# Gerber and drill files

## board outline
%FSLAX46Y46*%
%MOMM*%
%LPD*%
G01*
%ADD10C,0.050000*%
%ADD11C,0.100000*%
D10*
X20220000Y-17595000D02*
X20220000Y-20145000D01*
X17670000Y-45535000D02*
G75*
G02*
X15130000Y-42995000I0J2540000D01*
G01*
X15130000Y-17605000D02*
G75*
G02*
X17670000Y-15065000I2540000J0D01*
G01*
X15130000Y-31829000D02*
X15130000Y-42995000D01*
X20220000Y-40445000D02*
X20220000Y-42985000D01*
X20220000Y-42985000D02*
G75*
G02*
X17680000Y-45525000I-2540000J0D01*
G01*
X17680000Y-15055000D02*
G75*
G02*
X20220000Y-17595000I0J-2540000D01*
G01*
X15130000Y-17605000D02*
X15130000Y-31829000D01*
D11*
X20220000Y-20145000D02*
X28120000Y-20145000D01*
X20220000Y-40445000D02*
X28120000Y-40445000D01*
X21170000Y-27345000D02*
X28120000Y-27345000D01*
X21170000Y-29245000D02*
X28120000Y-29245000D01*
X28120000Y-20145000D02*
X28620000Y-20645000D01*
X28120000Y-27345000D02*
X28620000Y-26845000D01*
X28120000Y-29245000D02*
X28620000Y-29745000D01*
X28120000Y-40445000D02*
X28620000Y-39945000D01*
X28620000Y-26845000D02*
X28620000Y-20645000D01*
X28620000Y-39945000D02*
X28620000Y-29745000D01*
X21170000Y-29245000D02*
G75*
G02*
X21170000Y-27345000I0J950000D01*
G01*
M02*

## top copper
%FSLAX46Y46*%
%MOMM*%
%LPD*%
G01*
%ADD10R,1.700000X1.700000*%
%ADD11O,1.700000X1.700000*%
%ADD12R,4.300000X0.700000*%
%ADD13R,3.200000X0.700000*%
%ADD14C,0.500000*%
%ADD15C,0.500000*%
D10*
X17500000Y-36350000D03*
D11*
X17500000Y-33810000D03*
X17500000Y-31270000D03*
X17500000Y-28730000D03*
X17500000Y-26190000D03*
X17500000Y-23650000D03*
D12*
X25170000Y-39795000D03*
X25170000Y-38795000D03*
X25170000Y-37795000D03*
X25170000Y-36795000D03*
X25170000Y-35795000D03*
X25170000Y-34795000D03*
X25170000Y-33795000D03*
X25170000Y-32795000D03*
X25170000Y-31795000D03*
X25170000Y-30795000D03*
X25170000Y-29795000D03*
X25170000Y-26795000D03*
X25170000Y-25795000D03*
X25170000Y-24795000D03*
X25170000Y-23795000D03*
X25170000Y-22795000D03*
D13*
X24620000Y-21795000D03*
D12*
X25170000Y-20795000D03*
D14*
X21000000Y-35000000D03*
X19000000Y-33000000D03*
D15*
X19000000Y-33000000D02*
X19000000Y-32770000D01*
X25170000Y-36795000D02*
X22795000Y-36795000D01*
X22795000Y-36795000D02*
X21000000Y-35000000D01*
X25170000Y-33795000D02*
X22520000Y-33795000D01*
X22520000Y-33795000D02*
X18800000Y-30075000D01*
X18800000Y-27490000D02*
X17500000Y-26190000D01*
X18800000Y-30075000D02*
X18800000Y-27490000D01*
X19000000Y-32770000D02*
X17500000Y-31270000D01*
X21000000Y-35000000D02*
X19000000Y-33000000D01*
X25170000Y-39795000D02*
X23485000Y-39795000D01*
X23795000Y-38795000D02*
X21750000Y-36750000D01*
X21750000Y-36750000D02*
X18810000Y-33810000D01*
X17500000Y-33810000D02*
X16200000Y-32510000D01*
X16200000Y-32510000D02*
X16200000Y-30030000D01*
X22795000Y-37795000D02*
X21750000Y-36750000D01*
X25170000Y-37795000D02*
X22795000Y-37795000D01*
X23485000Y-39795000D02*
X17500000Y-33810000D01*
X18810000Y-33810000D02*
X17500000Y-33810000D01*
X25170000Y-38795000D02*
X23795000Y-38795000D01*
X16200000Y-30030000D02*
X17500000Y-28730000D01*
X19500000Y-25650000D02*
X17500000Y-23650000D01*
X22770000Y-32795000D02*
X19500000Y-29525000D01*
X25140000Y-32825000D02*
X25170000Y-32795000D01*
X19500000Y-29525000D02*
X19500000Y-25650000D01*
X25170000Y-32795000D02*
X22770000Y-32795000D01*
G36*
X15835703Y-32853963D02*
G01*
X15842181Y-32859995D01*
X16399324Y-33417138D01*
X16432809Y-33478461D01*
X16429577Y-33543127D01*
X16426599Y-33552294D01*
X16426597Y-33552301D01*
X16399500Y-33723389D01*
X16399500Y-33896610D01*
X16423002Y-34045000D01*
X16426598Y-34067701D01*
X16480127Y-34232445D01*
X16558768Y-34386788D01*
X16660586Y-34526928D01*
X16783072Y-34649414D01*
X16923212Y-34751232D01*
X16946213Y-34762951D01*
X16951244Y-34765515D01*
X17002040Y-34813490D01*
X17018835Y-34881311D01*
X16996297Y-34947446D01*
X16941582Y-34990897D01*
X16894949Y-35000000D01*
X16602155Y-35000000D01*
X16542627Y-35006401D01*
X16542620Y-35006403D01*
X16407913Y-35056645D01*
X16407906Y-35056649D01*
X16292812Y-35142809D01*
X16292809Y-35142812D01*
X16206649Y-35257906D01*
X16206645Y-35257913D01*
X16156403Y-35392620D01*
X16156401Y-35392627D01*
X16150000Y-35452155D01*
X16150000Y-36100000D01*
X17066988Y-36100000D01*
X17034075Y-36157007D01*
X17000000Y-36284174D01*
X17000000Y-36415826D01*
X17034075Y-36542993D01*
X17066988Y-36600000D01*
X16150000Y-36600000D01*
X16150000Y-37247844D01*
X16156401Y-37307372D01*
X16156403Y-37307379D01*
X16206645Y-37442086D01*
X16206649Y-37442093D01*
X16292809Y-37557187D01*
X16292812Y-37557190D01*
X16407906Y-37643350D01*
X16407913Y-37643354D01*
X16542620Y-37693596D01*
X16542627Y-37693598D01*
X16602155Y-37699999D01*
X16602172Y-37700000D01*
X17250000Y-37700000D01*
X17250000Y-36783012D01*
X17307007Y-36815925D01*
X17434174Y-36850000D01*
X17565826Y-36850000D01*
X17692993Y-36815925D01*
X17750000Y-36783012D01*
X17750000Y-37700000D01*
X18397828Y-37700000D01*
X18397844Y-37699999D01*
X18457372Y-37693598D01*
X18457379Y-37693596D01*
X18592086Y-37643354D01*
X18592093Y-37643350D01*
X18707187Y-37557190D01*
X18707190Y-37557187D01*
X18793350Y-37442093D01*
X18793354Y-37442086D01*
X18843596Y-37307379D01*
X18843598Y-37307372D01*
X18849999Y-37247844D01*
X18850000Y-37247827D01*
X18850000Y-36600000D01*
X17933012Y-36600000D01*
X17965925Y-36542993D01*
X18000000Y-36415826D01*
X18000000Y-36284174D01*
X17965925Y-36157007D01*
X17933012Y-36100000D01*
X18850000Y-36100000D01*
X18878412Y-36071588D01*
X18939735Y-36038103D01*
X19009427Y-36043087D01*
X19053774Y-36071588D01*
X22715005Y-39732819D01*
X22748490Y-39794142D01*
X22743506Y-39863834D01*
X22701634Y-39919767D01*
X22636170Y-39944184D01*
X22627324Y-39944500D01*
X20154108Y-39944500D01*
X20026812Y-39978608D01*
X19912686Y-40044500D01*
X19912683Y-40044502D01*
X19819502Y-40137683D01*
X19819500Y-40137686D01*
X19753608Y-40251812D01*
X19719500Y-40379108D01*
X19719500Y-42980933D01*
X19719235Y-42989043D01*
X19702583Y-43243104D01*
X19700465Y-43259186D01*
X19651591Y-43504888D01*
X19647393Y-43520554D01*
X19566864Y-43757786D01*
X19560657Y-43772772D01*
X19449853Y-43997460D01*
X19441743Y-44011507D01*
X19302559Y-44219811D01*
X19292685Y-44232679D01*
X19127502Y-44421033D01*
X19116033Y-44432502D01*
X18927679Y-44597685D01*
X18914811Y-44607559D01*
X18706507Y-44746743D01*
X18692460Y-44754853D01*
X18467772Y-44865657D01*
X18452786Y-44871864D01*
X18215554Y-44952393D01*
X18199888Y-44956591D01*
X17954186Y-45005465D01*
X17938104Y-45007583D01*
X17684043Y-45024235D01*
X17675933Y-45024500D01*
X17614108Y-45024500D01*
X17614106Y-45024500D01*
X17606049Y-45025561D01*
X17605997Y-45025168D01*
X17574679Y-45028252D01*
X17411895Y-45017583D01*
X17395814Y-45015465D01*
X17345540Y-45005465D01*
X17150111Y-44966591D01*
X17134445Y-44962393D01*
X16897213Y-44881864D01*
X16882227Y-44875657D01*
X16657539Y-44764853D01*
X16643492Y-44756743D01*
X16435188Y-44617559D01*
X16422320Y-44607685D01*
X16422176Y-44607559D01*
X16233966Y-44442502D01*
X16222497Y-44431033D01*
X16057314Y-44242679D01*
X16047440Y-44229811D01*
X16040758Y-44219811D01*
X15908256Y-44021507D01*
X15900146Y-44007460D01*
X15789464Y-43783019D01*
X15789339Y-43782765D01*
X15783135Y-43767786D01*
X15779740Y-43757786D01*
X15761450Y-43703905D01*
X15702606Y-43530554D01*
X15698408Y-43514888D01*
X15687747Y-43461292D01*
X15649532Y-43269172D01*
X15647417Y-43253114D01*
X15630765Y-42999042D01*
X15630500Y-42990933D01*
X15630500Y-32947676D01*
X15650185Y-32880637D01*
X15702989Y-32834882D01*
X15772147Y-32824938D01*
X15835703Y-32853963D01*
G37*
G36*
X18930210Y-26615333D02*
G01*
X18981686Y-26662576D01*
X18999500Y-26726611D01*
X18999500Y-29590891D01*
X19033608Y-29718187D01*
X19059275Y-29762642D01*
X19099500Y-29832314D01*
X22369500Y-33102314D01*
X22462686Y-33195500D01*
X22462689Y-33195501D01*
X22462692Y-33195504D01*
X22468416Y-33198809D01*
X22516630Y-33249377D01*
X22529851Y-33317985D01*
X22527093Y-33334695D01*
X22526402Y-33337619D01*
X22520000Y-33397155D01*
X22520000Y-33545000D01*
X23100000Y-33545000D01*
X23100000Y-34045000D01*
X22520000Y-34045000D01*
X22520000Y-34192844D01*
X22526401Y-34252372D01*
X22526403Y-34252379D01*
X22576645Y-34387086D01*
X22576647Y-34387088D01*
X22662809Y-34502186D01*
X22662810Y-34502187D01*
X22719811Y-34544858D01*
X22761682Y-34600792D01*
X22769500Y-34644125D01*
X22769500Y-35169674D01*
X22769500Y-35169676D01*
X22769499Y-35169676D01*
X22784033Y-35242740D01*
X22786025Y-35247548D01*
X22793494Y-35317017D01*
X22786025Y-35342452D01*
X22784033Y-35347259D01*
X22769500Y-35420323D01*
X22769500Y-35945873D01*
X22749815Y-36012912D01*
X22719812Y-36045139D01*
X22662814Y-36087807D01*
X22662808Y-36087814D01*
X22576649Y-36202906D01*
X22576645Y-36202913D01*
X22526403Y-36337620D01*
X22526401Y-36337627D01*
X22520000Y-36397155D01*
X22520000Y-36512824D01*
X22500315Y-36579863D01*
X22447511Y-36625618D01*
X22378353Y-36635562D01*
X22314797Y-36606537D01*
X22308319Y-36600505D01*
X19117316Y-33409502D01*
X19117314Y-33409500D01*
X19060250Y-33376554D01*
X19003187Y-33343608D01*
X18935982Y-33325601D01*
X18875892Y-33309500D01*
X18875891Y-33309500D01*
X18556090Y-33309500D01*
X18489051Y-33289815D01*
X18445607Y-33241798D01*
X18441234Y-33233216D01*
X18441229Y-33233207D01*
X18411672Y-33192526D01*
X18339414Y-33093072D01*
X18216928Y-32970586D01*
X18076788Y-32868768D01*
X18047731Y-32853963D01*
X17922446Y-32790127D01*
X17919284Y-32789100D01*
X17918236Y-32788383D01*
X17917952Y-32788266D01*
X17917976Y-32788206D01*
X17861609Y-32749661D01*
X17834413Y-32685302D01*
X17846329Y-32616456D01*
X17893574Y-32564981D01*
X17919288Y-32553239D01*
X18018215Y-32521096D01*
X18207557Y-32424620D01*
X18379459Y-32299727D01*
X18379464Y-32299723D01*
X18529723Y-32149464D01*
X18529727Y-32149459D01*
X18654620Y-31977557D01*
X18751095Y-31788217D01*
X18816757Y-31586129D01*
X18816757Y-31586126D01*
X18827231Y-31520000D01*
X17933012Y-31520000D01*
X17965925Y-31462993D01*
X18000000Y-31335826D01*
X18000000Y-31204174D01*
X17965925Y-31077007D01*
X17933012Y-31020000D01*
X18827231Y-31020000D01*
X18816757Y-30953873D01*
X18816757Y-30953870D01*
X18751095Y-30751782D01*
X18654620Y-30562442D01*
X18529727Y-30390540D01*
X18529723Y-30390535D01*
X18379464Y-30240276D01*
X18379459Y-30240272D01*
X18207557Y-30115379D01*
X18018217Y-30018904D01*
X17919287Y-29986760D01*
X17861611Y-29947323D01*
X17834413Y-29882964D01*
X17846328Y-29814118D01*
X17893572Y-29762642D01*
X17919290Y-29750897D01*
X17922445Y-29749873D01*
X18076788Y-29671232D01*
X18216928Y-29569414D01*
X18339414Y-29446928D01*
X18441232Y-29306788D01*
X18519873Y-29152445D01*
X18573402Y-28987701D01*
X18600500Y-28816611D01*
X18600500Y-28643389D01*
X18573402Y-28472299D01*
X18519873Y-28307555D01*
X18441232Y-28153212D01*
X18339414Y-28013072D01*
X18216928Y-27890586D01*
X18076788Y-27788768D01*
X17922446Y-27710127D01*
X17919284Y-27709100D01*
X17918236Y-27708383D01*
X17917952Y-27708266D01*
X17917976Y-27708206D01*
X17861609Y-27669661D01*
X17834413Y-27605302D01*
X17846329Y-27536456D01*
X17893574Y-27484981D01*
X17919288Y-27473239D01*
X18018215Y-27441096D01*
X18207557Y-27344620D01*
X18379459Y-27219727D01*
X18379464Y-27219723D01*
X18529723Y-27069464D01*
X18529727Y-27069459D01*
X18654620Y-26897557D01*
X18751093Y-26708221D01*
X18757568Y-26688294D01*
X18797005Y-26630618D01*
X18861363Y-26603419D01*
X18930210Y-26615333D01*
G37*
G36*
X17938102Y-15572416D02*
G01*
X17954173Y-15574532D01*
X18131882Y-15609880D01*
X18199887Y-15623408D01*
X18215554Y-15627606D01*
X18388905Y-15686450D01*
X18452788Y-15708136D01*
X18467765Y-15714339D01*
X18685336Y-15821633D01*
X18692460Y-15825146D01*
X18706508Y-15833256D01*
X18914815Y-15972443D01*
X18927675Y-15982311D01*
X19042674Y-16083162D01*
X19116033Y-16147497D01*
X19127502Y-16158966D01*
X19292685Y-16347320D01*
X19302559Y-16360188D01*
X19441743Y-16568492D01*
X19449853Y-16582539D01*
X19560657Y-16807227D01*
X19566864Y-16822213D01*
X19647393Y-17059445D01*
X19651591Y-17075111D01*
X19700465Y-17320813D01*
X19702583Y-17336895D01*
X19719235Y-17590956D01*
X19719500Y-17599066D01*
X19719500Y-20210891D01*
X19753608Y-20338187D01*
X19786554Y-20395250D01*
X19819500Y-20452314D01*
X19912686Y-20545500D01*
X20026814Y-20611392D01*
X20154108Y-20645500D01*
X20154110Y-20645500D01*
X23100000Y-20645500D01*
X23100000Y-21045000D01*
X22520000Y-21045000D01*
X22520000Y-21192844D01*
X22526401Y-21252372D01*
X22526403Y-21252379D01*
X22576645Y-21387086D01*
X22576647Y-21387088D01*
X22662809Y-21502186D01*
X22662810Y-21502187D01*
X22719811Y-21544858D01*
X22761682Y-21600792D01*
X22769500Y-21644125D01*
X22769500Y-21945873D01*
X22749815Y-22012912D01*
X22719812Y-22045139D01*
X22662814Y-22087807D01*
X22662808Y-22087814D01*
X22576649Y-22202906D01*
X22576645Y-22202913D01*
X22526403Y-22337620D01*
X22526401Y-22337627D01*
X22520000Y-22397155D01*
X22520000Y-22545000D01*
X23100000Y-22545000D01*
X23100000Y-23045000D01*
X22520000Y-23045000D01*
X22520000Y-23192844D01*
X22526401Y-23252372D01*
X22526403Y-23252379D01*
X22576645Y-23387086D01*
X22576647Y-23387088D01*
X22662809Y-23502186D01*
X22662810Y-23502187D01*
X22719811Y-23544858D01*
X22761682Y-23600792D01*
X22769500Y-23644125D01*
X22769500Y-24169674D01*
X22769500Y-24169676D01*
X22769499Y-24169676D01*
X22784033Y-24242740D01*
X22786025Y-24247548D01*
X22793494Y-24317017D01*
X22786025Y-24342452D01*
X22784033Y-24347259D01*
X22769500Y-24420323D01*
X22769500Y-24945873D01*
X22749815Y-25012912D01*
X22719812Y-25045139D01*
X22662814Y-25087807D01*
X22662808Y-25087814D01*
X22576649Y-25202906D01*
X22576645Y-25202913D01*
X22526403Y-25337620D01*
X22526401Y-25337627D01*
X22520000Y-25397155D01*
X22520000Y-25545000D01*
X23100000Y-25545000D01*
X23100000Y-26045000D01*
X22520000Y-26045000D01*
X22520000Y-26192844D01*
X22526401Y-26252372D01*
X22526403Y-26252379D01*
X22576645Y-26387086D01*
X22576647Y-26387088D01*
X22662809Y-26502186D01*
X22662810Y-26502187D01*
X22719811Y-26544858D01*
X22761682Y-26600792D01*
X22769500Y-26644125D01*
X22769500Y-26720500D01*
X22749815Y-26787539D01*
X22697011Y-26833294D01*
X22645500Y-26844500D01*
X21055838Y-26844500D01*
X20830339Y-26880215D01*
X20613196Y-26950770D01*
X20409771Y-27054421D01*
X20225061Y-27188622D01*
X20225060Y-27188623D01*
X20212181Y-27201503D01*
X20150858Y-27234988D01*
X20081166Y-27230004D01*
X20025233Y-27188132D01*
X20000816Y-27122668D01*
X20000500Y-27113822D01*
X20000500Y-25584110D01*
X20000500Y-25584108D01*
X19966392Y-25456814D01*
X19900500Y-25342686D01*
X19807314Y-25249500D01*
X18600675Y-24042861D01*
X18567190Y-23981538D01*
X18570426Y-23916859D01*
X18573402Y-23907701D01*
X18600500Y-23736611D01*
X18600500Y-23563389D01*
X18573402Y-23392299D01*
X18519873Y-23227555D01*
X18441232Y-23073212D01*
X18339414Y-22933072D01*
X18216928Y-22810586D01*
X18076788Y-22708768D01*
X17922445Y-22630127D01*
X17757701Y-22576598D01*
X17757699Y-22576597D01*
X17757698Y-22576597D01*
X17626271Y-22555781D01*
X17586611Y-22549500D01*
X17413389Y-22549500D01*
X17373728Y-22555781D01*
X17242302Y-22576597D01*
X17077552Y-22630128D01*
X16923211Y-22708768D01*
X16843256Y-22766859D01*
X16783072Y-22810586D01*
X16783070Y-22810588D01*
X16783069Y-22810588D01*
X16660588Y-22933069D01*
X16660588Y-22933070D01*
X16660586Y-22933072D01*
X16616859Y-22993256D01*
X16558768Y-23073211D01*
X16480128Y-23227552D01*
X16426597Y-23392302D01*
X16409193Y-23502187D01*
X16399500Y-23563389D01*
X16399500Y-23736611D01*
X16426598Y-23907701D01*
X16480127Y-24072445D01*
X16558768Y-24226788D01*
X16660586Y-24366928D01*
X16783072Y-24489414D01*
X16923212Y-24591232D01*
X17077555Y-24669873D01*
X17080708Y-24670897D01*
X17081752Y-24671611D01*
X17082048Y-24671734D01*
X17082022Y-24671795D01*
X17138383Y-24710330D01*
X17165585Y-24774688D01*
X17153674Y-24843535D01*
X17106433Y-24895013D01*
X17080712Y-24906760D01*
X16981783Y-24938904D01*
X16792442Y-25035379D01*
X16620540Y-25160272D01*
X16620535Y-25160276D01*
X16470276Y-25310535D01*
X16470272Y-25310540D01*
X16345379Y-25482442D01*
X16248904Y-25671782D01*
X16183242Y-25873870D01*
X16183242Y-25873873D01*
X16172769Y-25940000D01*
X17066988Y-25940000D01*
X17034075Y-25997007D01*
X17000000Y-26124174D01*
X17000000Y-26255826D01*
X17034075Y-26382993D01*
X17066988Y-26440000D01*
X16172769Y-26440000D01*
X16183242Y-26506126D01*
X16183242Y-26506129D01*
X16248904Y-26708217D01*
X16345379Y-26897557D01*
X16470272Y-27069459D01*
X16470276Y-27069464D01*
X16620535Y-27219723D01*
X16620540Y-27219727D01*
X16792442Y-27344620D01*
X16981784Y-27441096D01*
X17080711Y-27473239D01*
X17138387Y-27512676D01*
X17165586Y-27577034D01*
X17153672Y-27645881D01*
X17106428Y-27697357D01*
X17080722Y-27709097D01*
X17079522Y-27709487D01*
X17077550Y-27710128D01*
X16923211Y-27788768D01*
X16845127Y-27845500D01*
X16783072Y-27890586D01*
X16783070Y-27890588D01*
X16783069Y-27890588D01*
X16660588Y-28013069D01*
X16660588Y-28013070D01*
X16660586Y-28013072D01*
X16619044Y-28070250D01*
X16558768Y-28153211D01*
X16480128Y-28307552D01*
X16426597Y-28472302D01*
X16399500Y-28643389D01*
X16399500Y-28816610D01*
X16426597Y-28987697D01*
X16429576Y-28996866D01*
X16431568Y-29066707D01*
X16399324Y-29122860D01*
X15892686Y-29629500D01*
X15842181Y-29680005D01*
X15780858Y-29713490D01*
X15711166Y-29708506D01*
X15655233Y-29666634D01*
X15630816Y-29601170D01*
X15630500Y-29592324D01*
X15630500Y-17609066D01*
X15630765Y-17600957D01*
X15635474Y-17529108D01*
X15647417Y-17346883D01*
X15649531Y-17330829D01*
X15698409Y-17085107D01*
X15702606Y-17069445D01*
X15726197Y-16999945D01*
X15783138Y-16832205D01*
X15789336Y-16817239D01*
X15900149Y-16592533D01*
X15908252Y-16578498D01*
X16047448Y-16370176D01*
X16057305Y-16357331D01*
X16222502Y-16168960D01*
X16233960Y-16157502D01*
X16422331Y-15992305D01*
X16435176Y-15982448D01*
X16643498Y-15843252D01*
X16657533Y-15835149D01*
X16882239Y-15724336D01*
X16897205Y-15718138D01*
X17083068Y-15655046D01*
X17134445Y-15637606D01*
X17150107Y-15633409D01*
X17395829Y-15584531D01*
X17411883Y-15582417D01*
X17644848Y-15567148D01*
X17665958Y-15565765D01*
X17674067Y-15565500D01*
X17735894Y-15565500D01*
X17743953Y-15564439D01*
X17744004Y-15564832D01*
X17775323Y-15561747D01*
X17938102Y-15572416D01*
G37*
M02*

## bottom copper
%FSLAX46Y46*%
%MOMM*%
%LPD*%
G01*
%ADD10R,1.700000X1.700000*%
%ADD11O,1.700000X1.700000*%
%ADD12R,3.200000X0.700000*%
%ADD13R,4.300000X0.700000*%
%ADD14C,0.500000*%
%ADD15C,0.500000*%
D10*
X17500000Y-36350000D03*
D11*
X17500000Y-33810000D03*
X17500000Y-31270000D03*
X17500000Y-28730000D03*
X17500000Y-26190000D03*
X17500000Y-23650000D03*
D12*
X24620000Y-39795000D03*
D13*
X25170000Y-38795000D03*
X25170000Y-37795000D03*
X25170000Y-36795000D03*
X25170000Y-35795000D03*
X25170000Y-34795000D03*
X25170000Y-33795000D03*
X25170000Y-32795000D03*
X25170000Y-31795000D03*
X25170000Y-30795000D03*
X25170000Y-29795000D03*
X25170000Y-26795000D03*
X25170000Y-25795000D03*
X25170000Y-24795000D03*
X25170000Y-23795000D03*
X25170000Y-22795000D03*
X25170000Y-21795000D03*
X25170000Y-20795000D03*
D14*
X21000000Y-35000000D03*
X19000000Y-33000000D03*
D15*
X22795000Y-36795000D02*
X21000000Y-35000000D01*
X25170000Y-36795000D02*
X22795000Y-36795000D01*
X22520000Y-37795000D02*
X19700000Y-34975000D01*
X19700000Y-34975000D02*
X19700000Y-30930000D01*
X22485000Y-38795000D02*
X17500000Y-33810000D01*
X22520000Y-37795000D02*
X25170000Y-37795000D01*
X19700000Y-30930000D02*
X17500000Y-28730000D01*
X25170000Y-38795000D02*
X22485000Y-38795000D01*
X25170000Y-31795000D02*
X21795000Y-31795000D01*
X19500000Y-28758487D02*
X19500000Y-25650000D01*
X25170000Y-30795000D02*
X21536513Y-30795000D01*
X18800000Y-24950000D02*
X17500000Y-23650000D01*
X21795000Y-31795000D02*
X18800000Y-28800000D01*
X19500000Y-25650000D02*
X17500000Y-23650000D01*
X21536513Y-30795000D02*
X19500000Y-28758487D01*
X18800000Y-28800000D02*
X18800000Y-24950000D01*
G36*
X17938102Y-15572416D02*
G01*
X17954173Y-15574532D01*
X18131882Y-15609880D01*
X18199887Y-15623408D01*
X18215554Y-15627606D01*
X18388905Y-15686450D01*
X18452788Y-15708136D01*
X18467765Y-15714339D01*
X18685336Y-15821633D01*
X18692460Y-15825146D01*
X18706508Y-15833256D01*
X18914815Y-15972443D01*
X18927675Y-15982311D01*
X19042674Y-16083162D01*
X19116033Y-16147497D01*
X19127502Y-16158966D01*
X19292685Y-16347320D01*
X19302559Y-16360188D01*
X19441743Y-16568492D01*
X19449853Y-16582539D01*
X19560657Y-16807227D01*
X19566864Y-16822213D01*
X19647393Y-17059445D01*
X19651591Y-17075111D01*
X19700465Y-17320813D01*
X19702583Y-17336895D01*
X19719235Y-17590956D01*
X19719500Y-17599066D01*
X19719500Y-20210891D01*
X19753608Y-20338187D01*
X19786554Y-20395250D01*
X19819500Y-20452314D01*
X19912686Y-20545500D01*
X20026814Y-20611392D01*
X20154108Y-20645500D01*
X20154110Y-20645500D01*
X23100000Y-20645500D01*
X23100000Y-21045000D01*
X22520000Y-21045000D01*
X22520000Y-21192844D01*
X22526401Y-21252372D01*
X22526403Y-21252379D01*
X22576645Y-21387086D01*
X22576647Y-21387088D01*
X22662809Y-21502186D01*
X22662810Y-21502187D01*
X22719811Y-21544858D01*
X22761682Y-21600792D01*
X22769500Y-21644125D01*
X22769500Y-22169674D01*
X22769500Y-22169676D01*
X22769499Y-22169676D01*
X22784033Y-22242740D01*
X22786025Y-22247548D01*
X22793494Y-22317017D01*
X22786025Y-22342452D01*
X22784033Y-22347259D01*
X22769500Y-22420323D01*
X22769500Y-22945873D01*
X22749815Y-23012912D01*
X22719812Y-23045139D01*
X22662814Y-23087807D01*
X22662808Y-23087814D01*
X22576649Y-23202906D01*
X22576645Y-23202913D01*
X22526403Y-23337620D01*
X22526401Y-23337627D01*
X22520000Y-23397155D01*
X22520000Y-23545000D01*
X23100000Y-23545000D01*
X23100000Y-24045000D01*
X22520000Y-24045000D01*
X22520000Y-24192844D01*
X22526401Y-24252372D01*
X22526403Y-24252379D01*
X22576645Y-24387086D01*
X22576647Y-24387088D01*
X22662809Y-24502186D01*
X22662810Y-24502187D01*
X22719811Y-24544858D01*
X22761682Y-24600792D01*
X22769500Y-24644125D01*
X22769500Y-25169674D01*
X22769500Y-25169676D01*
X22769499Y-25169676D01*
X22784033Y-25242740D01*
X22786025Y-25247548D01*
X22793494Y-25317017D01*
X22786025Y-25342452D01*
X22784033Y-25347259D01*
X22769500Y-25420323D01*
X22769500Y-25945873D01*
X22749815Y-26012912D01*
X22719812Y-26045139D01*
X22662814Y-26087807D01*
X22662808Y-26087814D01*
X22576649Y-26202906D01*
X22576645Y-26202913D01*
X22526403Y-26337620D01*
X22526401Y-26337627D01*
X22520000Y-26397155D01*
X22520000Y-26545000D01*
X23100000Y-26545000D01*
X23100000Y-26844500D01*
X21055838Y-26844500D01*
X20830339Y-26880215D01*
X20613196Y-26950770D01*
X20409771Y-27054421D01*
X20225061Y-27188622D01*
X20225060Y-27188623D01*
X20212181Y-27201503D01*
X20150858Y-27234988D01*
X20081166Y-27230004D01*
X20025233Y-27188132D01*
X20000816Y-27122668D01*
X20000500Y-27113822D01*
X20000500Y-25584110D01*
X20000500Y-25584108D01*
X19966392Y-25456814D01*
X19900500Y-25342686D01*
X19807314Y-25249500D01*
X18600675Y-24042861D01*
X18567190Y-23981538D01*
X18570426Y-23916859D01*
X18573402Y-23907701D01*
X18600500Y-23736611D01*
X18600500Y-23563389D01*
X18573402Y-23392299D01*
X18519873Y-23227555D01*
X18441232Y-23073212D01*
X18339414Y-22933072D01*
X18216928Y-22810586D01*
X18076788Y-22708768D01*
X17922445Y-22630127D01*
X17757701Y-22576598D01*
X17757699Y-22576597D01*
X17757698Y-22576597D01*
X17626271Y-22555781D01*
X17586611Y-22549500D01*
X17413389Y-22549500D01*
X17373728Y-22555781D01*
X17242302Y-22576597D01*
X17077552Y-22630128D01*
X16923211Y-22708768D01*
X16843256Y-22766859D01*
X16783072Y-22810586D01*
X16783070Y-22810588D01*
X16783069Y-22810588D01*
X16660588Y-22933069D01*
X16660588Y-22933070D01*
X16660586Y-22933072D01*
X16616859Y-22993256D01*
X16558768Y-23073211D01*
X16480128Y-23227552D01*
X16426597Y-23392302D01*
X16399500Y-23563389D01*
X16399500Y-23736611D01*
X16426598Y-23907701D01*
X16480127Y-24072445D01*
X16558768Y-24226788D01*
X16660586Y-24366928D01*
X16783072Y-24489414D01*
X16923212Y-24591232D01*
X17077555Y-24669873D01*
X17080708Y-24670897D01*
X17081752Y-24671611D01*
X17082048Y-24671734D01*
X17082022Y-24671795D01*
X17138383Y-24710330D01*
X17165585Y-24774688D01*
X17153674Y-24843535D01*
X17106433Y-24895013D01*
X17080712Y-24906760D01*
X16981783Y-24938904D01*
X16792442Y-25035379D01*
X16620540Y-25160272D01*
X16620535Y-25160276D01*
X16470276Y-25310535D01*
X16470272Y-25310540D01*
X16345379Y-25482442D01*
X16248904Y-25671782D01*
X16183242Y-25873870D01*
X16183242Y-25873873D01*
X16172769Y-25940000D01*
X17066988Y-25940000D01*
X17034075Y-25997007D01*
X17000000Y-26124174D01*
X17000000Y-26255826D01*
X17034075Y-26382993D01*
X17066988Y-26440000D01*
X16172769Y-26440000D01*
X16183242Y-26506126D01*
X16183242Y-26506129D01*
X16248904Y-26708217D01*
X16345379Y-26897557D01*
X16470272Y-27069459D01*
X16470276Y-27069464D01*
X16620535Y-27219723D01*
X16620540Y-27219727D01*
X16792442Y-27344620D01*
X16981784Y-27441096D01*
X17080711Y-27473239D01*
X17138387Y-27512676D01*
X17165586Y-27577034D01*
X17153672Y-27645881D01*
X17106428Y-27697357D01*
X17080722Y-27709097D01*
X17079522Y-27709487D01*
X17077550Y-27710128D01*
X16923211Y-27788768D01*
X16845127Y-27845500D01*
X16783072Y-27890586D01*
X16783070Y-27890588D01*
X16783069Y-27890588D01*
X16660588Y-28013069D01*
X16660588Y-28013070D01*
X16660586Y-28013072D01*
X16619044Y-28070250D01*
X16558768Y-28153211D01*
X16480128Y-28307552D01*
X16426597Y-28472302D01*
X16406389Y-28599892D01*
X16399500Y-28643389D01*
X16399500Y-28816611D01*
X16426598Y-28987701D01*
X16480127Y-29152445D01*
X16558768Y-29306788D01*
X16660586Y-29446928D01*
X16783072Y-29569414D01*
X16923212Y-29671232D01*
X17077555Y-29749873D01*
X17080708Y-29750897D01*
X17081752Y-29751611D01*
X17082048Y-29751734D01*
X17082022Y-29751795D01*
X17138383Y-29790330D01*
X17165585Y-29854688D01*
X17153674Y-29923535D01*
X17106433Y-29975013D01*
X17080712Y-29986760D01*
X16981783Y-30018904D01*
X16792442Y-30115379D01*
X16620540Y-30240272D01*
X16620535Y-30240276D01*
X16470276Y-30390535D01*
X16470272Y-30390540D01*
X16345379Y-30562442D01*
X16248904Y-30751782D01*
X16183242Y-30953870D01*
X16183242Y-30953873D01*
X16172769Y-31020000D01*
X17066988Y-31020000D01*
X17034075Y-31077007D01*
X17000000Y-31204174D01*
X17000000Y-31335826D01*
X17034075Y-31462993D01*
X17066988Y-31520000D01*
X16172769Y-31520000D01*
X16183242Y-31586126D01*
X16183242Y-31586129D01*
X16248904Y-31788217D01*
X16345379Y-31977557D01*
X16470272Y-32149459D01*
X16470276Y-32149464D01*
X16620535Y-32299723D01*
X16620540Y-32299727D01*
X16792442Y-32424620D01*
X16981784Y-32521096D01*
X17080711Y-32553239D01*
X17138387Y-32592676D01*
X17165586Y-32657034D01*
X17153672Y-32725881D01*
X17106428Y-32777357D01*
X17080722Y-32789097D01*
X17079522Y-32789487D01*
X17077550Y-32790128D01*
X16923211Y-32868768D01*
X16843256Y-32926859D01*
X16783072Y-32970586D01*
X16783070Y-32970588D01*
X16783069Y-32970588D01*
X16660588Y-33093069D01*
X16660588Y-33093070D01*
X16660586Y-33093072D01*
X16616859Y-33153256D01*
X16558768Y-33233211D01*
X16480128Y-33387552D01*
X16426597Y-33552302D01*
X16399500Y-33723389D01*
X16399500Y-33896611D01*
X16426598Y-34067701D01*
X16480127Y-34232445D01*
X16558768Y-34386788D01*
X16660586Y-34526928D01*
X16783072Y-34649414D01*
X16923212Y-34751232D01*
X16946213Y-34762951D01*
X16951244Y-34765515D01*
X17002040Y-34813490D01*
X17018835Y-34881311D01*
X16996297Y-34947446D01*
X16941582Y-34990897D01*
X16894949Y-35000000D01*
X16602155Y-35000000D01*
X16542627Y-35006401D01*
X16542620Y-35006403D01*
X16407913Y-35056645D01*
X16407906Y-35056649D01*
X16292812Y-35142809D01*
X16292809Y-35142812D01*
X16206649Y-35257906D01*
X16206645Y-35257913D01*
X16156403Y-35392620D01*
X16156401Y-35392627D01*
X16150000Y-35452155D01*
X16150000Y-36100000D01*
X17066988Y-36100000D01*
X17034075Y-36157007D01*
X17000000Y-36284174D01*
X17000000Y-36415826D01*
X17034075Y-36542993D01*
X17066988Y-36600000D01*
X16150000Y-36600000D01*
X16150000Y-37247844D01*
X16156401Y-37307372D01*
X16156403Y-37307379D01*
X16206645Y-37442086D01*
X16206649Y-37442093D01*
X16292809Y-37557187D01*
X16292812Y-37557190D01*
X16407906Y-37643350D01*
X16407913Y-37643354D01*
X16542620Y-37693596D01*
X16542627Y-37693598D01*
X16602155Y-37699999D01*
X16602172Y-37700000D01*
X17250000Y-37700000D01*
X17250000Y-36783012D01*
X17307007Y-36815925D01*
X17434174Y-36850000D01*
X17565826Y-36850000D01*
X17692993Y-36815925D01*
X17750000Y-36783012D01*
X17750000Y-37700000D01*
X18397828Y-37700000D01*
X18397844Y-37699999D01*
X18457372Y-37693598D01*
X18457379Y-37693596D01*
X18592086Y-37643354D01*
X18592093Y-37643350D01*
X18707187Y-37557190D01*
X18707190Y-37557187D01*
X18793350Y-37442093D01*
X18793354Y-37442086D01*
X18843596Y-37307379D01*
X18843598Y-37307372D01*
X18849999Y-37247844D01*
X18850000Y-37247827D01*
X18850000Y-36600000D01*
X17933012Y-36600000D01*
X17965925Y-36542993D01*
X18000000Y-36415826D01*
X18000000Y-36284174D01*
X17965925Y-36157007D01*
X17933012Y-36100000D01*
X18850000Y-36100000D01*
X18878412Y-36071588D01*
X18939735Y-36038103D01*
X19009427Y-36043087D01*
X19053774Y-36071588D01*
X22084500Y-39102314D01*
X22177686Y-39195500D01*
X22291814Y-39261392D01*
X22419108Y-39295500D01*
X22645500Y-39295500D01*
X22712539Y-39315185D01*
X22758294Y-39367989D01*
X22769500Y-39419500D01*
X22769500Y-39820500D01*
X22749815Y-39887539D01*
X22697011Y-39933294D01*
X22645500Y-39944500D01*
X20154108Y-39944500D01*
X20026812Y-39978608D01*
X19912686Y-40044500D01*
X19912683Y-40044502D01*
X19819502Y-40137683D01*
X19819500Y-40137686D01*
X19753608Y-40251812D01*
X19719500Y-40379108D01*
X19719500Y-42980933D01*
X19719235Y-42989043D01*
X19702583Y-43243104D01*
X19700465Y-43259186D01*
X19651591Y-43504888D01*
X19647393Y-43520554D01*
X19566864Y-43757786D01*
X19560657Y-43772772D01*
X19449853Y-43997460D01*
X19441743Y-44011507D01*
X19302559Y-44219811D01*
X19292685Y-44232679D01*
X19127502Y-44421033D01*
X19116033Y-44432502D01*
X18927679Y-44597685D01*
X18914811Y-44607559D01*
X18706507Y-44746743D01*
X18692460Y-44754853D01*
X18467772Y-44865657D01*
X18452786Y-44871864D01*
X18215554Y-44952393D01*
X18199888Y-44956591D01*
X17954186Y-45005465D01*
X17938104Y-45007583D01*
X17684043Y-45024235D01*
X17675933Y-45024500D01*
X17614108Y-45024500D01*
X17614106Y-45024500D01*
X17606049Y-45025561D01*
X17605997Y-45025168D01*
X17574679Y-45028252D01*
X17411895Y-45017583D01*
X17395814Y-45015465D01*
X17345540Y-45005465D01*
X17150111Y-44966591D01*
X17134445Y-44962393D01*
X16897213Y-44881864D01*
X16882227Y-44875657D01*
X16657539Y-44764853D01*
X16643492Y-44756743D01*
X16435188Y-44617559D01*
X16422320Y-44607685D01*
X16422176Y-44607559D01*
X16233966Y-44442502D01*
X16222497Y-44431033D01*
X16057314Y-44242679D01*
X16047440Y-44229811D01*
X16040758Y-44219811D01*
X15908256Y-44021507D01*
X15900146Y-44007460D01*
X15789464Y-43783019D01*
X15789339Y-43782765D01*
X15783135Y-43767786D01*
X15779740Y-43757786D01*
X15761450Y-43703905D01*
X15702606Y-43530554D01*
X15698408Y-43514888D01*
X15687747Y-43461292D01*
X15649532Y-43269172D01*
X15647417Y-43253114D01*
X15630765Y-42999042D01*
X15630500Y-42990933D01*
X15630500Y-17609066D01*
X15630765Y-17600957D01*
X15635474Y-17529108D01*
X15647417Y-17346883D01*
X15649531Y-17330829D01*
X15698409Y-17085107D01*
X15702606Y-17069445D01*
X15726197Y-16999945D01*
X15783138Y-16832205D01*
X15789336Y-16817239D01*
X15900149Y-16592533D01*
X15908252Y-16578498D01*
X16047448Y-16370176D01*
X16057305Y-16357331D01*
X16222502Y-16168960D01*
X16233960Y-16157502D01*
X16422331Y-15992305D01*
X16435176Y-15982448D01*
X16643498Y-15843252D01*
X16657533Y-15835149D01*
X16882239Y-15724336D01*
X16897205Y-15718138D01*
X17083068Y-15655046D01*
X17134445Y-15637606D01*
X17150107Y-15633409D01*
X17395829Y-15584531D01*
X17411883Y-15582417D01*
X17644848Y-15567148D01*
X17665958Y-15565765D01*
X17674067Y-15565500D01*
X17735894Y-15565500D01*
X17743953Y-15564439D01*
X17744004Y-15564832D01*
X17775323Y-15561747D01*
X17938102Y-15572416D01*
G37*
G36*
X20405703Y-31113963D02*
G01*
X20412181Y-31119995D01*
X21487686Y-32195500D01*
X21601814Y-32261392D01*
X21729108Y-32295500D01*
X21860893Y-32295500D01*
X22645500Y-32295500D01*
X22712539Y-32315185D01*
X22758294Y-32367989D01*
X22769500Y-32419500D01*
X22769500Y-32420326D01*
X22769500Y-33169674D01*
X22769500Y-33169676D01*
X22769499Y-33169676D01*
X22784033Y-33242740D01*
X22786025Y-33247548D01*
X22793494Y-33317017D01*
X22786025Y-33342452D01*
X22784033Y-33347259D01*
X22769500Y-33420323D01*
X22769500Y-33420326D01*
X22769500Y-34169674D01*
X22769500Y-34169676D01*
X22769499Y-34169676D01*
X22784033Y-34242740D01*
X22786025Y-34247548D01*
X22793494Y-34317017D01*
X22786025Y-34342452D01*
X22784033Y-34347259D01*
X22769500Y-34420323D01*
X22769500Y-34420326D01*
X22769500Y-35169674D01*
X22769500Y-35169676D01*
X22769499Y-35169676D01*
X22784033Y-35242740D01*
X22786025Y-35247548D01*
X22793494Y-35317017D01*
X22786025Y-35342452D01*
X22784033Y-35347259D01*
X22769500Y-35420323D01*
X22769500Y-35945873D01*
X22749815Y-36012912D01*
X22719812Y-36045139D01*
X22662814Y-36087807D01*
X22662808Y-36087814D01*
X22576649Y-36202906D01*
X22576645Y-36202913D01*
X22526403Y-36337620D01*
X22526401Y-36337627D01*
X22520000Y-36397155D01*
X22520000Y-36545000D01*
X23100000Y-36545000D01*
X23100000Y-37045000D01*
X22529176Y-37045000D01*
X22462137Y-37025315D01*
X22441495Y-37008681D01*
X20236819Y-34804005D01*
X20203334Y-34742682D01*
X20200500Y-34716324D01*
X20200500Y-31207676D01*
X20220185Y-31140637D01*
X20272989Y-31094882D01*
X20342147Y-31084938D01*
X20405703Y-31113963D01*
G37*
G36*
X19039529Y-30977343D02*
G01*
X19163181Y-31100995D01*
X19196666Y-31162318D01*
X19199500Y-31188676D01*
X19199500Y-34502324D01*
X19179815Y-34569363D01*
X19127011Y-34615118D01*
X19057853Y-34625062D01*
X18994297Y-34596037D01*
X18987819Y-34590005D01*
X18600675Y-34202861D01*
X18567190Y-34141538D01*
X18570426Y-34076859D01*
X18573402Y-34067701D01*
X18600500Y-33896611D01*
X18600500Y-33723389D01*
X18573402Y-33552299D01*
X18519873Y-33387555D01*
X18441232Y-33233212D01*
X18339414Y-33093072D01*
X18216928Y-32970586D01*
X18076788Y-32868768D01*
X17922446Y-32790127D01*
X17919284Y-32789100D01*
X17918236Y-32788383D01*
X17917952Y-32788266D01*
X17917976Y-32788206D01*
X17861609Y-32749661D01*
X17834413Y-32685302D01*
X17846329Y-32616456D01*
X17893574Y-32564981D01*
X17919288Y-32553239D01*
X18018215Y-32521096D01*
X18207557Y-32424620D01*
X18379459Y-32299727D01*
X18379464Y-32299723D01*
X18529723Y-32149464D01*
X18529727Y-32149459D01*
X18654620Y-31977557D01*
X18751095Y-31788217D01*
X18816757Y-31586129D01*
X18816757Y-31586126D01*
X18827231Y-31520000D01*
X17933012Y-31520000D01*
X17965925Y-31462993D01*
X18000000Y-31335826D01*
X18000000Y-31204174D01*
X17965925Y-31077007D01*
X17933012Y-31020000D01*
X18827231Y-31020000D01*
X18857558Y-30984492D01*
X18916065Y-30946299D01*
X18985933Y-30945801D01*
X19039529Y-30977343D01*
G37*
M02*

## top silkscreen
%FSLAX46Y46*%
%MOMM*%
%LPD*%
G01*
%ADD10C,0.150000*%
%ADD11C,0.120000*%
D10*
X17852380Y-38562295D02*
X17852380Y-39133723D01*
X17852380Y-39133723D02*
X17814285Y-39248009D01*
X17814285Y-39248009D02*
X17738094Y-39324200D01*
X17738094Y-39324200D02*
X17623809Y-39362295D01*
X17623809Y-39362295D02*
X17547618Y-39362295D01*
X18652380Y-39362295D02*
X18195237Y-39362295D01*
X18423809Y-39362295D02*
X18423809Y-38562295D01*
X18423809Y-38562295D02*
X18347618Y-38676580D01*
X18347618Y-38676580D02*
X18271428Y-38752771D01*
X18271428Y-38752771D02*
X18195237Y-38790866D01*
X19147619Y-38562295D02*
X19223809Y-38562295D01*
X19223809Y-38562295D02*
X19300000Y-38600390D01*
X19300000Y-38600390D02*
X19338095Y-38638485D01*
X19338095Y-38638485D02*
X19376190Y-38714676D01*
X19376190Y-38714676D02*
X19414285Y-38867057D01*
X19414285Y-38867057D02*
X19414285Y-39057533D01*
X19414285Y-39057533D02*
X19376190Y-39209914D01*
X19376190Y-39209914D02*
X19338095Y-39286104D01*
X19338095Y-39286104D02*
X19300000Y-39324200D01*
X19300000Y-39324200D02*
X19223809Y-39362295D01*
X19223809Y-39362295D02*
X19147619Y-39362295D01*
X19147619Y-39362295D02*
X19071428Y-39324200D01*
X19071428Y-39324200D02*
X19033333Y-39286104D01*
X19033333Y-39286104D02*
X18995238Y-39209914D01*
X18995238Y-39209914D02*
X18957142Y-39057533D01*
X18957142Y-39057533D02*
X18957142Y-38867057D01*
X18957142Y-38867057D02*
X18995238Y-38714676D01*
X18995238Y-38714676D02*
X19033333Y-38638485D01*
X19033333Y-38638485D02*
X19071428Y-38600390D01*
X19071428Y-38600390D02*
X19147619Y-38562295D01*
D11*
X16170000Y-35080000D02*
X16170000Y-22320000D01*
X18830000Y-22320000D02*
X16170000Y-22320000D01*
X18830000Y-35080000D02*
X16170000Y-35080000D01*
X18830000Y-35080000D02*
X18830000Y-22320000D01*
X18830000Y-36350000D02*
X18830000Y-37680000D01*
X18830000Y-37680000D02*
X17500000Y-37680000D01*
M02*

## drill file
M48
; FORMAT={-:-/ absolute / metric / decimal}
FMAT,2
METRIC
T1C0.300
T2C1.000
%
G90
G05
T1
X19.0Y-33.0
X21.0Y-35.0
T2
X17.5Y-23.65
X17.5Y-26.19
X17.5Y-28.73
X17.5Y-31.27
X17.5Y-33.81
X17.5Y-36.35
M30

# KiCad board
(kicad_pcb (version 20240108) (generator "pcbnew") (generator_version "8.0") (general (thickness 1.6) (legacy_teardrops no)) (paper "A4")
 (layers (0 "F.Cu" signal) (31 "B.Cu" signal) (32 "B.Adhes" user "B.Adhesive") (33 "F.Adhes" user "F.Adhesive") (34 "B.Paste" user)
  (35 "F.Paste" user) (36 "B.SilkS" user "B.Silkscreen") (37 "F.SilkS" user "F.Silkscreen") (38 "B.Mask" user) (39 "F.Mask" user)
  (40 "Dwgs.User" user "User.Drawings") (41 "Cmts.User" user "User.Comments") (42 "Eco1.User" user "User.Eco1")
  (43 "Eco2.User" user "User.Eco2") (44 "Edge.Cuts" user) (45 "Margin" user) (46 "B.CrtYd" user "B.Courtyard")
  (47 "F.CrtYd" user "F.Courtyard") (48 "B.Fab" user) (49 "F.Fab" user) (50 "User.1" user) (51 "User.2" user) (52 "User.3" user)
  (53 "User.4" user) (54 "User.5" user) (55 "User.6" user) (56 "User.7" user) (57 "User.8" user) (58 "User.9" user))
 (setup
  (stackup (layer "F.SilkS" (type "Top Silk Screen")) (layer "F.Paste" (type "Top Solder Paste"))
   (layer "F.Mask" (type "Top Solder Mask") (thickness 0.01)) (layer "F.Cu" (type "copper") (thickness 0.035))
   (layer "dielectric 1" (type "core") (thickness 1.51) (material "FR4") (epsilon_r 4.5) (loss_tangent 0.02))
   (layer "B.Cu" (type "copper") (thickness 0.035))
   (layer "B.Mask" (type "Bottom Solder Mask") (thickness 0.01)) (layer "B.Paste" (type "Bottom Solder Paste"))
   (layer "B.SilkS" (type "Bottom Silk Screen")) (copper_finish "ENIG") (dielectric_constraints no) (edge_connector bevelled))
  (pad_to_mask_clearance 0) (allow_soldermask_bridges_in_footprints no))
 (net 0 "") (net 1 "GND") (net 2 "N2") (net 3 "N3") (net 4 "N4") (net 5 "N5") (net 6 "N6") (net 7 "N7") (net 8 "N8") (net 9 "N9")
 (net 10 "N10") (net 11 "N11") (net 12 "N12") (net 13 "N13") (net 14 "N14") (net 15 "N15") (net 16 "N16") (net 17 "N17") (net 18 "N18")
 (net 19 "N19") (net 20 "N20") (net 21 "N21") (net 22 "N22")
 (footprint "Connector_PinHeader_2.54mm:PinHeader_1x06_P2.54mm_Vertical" (layer "F.Cu") (at 17.5 36.35 180)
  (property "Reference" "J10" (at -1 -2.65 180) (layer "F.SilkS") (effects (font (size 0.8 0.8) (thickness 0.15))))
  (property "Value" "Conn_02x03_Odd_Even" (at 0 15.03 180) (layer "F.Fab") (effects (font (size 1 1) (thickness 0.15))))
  (fp_line (start 1.33 1.27) (end 1.33 14.03) (stroke (width 0.12) (type solid)) (layer "F.SilkS"))
  (fp_line (start -1.33 14.03) (end 1.33 14.03) (stroke (width 0.12) (type solid)) (layer "F.SilkS"))
  (fp_line (start -1.33 1.27) (end 1.33 1.27) (stroke (width 0.12) (type solid)) (layer "F.SilkS"))
  (fp_line (start -1.33 1.27) (end -1.33 14.03) (stroke (width 0.12) (type solid)) (layer "F.SilkS"))
  (fp_line (start -1.33 0) (end -1.33 -1.33) (stroke (width 0.12) (type solid)) (layer "F.SilkS"))
  (fp_line (start -1.33 -1.33) (end 0 -1.33) (stroke (width 0.12) (type solid)) (layer "F.SilkS"))
  (pad "1" thru_hole rect (at 0 0 180) (size 1.7 1.7) (drill 1) (layers "*.Cu" "*.Mask") (remove_unused_layers no) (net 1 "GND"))
  (pad "2" thru_hole oval (at 0 2.54 180) (size 1.7 1.7) (drill 1) (layers "*.Cu" "*.Mask") (remove_unused_layers no) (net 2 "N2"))
  (pad "3" thru_hole oval (at 0 5.08 180) (size 1.7 1.7) (drill 1) (layers "*.Cu" "*.Mask") (remove_unused_layers no) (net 1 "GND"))
  (pad "4" thru_hole oval (at 0 7.62 180) (size 1.7 1.7) (drill 1) (layers "*.Cu" "*.Mask") (remove_unused_layers no) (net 2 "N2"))
  (pad "5" thru_hole oval (at 0 10.16 180) (size 1.7 1.7) (drill 1) (layers "*.Cu" "*.Mask") (remove_unused_layers no) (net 1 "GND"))
  (pad "6" thru_hole oval (at 0 12.7 180) (size 1.7 1.7) (drill 1) (layers "*.Cu" "*.Mask") (remove_unused_layers no) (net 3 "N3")))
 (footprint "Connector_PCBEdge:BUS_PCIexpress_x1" (layer "F.Cu") (at 25.17 39.795 90)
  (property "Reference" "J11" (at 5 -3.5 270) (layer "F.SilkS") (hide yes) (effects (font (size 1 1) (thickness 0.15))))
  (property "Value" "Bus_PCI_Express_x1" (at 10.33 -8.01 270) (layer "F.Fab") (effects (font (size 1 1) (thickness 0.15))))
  (fp_line (start 19.65 -4.95) (end 19.65 2.95) (stroke (width 0.1) (type solid)) (layer "Edge.Cuts"))
  (fp_line (start -0.65 -4.95) (end -0.65 2.95) (stroke (width 0.1) (type solid)) (layer "Edge.Cuts"))
  (fp_line (start 12.45 -4) (end 12.45 2.95) (stroke (width 0.1) (type solid)) (layer "Edge.Cuts"))
  (fp_line (start 10.55 -4) (end 10.55 2.95) (stroke (width 0.1) (type solid)) (layer "Edge.Cuts"))
  (fp_line (start 19.65 2.95) (end 19.15 3.45) (stroke (width 0.1) (type solid)) (layer "Edge.Cuts"))
  (fp_line (start 12.45 2.95) (end 12.95 3.45) (stroke (width 0.1) (type solid)) (layer "Edge.Cuts"))
  (fp_line (start 10.55 2.95) (end 10.05 3.45) (stroke (width 0.1) (type solid)) (layer "Edge.Cuts"))
  (fp_line (start -0.65 2.95) (end -0.15 3.45) (stroke (width 0.1) (type solid)) (layer "Edge.Cuts"))
  (fp_line (start 12.95 3.45) (end 19.15 3.45) (stroke (width 0.1) (type solid)) (layer "Edge.Cuts"))
  (fp_line (start -0.15 3.45) (end 10.05 3.45) (stroke (width 0.1) (type solid)) (layer "Edge.Cuts"))
  (fp_arc (start 10.55 -4) (mid 11.5 -4.95) (end 12.45 -4) (stroke (width 0.1) (type solid)) (layer "Edge.Cuts"))
  (pad "A1" connect rect (at 0 -0.55 90) (size 0.7 3.2) (layers "B.Cu" "B.Mask") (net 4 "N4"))
  (pad "A2" connect rect (at 1 0 90) (size 0.7 4.3) (layers "B.Cu" "B.Mask") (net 2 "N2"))
  (pad "A3" connect rect (at 2 0 90) (size 0.7 4.3) (layers "B.Cu" "B.Mask") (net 2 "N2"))
  (pad "A4" connect rect (at 3 0 90) (size 0.7 4.3) (layers "B.Cu" "B.Mask") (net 1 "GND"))
  (pad "A5" connect rect (at 4 0 90) (size 0.7 4.3) (layers "B.Cu" "B.Mask") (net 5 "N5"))
  (pad "A6" connect rect (at 5 0 90) (size 0.7 4.3) (layers "B.Cu" "B.Mask") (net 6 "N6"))
  (pad "A7" connect rect (at 6 0 90) (size 0.7 4.3) (layers "B.Cu" "B.Mask") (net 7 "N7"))
  (pad "A8" connect rect (at 7 0 90) (size 0.7 4.3) (layers "B.Cu" "B.Mask") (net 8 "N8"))
  (pad "A9" connect rect (at 8 0 90) (size 0.7 4.3) (layers "B.Cu" "B.Mask") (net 3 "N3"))
  (pad "A10" connect rect (at 9 0 90) (size 0.7 4.3) (layers "B.Cu" "B.Mask") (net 3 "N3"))
  (pad "A11" connect rect (at 10 0 90) (size 0.7 4.3) (layers "B.Cu" "B.Mask") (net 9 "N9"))
  (pad "A12" connect rect (at 13 0 90) (size 0.7 4.3) (layers "B.Cu" "B.Mask") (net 1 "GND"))
  (pad "A13" connect rect (at 14 0 90) (size 0.7 4.3) (layers "B.Cu" "B.Mask") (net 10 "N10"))
  (pad "A14" connect rect (at 15 0 90) (size 0.7 4.3) (layers "B.Cu" "B.Mask") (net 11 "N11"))
  (pad "A15" connect rect (at 16 0 90) (size 0.7 4.3) (layers "B.Cu" "B.Mask") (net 1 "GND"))
  (pad "A16" connect rect (at 17 0 90) (size 0.7 4.3) (layers "B.Cu" "B.Mask") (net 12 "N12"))
  (pad "A17" connect rect (at 18 0 90) (size 0.7 4.3) (layers "B.Cu" "B.Mask") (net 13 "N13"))
  (pad "A18" connect rect (at 19 0 90) (size 0.7 4.3) (layers "B.Cu" "B.Mask") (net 1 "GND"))
  (pad "B1" connect rect (at 0 0 90) (size 0.7 4.3) (layers "F.Cu" "F.Mask") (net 2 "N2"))
  (pad "B2" connect rect (at 1 0 90) (size 0.7 4.3) (layers "F.Cu" "F.Mask") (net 2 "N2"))
  (pad "B3" connect rect (at 2 0 90) (size 0.7 4.3) (layers "F.Cu" "F.Mask") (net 2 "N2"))
  (pad "B4" connect rect (at 3 0 90) (size 0.7 4.3) (layers "F.Cu" "F.Mask") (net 1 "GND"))
  (pad "B5" connect rect (at 4 0 90) (size 0.7 4.3) (layers "F.Cu" "F.Mask") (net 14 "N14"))
  (pad "B6" connect rect (at 5 0 90) (size 0.7 4.3) (layers "F.Cu" "F.Mask") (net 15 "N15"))
  (pad "B7" connect rect (at 6 0 90) (size 0.7 4.3) (layers "F.Cu" "F.Mask") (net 1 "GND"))
  (pad "B8" connect rect (at 7 0 90) (size 0.7 4.3) (layers "F.Cu" "F.Mask") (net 3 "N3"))
  (pad "B9" connect rect (at 8 0 90) (size 0.7 4.3) (layers "F.Cu" "F.Mask") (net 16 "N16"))
  (pad "B10" connect rect (at 9 0 90) (size 0.7 4.3) (layers "F.Cu" "F.Mask") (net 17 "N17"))
  (pad "B11" connect rect (at 10 0 90) (size 0.7 4.3) (layers "F.Cu" "F.Mask") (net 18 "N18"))
  (pad "B12" connect rect (at 13 0 90) (size 0.7 4.3) (layers "F.Cu" "F.Mask") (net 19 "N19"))
  (pad "B13" connect rect (at 14 0 90) (size 0.7 4.3) (layers "F.Cu" "F.Mask") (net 1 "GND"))
  (pad "B14" connect rect (at 15 0 90) (size 0.7 4.3) (layers "F.Cu" "F.Mask") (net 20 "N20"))
  (pad "B15" connect rect (at 16 0 90) (size 0.7 4.3) (layers "F.Cu" "F.Mask") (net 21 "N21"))
  (pad "B16" connect rect (at 17 0 90) (size 0.7 4.3) (layers "F.Cu" "F.Mask") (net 1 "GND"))
  (pad "B17" connect rect (at 18 -0.55 90) (size 0.7 3.2) (layers "F.Cu" "F.Mask") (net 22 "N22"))
  (pad "B18" connect rect (at 19 0 90) (size 0.7 4.3) (layers "F.Cu" "F.Mask") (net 1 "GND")))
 (gr_line (start 20.22 17.595) (end 20.22 20.145) (stroke (width 0.05) (type default)) (layer "Edge.Cuts"))
 (gr_arc (start 17.67 45.535) (mid 15.873949 44.791051) (end 15.13 42.995) (stroke (width 0.05) (type default)) (layer "Edge.Cuts"))
 (gr_arc (start 15.13 17.605) (mid 15.873949 15.808949) (end 17.67 15.065) (stroke (width 0.05) (type default)) (layer "Edge.Cuts"))
 (gr_line (start 15.13 31.829) (end 15.13 42.995) (stroke (width 0.05) (type default)) (layer "Edge.Cuts"))
 (gr_line (start 20.22 40.445) (end 20.22 42.985) (stroke (width 0.05) (type default)) (layer "Edge.Cuts"))
 (gr_arc (start 20.22 42.985) (mid 19.476051 44.781051) (end 17.68 45.525) (stroke (width 0.05) (type default)) (layer "Edge.Cuts"))
 (gr_arc (start 17.68 15.055) (mid 19.476051 15.798949) (end 20.22 17.595) (stroke (width 0.05) (type default)) (layer "Edge.Cuts"))
 (gr_line (start 15.13 17.605) (end 15.13 31.829) (stroke (width 0.05) (type default)) (layer "Edge.Cuts"))
 (segment (start 19 33) (end 19 32.77) (width 0.5) (layer "F.Cu") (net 1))
 (segment (start 25.17 36.795) (end 22.795 36.795) (width 0.5) (layer "F.Cu") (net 1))
 (segment (start 22.795 36.795) (end 21 35) (width 0.5) (layer "F.Cu") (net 1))
 (segment (start 25.17 33.795) (end 22.52 33.795) (width 0.5) (layer "F.Cu") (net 1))
 (segment (start 22.52 33.795) (end 18.8 30.075) (width 0.5) (layer "F.Cu") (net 1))
 (segment (start 18.8 27.49) (end 17.5 26.19) (width 0.5) (layer "F.Cu") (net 1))
 (segment (start 18.8 30.075) (end 18.8 27.49) (width 0.5) (layer "F.Cu") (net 1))
 (segment (start 19 32.77) (end 17.5 31.27) (width 0.5) (layer "F.Cu") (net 1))
 (segment (start 21 35) (end 19 33) (width 0.5) (layer "F.Cu") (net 1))
 (via (at 21 35) (size 0.5) (drill 0.3) (layers "F.Cu" "B.Cu") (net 1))
 (via (at 19 33) (size 0.5) (drill 0.3) (layers "F.Cu" "B.Cu") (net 1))
 (segment (start 22.795 36.795) (end 21 35) (width 0.5) (layer "B.Cu") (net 1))
 (segment (start 25.17 36.795) (end 22.795 36.795) (width 0.5) (layer "B.Cu") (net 1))
 (segment (start 25.17 39.795) (end 23.485 39.795) (width 0.5) (layer "F.Cu") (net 2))
 (segment (start 23.795 38.795) (end 21.75 36.75) (width 0.5) (layer "F.Cu") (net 2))
 (segment (start 21.75 36.75) (end 18.81 33.81) (width 0.5) (layer "F.Cu") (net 2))
 (segment (start 17.5 33.81) (end 16.2 32.51) (width 0.5) (layer "F.Cu") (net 2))
 (segment (start 16.2 32.51) (end 16.2 30.03) (width 0.5) (layer "F.Cu") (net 2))
 (segment (start 22.795 37.795) (end 21.75 36.75) (width 0.5) (layer "F.Cu") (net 2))
 (segment (start 25.17 37.795) (end 22.795 37.795) (width 0.5) (layer "F.Cu") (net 2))
 (segment (start 23.485 39.795) (end 17.5 33.81) (width 0.5) (layer "F.Cu") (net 2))
 (segment (start 18.81 33.81) (end 17.5 33.81) (width 0.5) (layer "F.Cu") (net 2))
 (segment (start 25.17 38.795) (end 23.795 38.795) (width 0.5) (layer "F.Cu") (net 2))
 (segment (start 16.2 30.03) (end 17.5 28.73) (width 0.5) (layer "F.Cu") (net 2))
 (segment (start 22.52 37.795) (end 19.7 34.975) (width 0.5) (layer "B.Cu") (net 2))
 (segment (start 19.7 34.975) (end 19.7 30.93) (width 0.5) (layer "B.Cu") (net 2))
 (segment (start 22.485 38.795) (end 17.5 33.81) (width 0.5) (layer "B.Cu") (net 2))
 (segment (start 22.52 37.795) (end 25.17 37.795) (width 0.5) (layer "B.Cu") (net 2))
 (segment (start 19.7 30.93) (end 17.5 28.73) (width 0.5) (layer "B.Cu") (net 2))
 (segment (start 25.17 38.795) (end 22.485 38.795) (width 0.5) (layer "B.Cu") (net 2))
 (segment (start 19.5 25.65) (end 17.5 23.65) (width 0.5) (layer "F.Cu") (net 3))
 (segment (start 22.77 32.795) (end 19.5 29.525) (width 0.5) (layer "F.Cu") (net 3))
 (segment (start 25.14 32.825) (end 25.17 32.795) (width 0.5) (layer "F.Cu") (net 3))
 (segment (start 19.5 29.525) (end 19.5 25.65) (width 0.5) (layer "F.Cu") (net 3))
 (segment (start 25.17 32.795) (end 22.77 32.795) (width 0.5) (layer "F.Cu") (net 3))
 (segment (start 25.17 31.795) (end 21.795 31.795) (width 0.5) (layer "B.Cu") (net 3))
 (segment (start 19.5 28.758487) (end 19.5 25.65) (width 0.5) (layer "B.Cu") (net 3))
 (segment (start 25.17 30.795) (end 21.536513 30.795) (width 0.5) (layer "B.Cu") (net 3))
 (segment (start 18.8 24.95) (end 17.5 23.65) (width 0.5) (layer "B.Cu") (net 3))
 (segment (start 21.795 31.795) (end 18.8 28.8) (width 0.5) (layer "B.Cu") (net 3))
 (segment (start 19.5 25.65) (end 17.5 23.65) (width 0.5) (layer "B.Cu") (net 3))
 (segment (start 21.536513 30.795) (end 19.5 28.758487) (width 0.5) (layer "B.Cu") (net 3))
 (segment (start 18.8 28.8) (end 18.8 24.95) (width 0.5) (layer "B.Cu") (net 3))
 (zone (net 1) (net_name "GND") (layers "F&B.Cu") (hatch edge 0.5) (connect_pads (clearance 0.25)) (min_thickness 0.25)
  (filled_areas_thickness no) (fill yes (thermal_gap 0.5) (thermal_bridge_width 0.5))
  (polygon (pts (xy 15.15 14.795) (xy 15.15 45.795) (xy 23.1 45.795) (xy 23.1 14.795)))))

